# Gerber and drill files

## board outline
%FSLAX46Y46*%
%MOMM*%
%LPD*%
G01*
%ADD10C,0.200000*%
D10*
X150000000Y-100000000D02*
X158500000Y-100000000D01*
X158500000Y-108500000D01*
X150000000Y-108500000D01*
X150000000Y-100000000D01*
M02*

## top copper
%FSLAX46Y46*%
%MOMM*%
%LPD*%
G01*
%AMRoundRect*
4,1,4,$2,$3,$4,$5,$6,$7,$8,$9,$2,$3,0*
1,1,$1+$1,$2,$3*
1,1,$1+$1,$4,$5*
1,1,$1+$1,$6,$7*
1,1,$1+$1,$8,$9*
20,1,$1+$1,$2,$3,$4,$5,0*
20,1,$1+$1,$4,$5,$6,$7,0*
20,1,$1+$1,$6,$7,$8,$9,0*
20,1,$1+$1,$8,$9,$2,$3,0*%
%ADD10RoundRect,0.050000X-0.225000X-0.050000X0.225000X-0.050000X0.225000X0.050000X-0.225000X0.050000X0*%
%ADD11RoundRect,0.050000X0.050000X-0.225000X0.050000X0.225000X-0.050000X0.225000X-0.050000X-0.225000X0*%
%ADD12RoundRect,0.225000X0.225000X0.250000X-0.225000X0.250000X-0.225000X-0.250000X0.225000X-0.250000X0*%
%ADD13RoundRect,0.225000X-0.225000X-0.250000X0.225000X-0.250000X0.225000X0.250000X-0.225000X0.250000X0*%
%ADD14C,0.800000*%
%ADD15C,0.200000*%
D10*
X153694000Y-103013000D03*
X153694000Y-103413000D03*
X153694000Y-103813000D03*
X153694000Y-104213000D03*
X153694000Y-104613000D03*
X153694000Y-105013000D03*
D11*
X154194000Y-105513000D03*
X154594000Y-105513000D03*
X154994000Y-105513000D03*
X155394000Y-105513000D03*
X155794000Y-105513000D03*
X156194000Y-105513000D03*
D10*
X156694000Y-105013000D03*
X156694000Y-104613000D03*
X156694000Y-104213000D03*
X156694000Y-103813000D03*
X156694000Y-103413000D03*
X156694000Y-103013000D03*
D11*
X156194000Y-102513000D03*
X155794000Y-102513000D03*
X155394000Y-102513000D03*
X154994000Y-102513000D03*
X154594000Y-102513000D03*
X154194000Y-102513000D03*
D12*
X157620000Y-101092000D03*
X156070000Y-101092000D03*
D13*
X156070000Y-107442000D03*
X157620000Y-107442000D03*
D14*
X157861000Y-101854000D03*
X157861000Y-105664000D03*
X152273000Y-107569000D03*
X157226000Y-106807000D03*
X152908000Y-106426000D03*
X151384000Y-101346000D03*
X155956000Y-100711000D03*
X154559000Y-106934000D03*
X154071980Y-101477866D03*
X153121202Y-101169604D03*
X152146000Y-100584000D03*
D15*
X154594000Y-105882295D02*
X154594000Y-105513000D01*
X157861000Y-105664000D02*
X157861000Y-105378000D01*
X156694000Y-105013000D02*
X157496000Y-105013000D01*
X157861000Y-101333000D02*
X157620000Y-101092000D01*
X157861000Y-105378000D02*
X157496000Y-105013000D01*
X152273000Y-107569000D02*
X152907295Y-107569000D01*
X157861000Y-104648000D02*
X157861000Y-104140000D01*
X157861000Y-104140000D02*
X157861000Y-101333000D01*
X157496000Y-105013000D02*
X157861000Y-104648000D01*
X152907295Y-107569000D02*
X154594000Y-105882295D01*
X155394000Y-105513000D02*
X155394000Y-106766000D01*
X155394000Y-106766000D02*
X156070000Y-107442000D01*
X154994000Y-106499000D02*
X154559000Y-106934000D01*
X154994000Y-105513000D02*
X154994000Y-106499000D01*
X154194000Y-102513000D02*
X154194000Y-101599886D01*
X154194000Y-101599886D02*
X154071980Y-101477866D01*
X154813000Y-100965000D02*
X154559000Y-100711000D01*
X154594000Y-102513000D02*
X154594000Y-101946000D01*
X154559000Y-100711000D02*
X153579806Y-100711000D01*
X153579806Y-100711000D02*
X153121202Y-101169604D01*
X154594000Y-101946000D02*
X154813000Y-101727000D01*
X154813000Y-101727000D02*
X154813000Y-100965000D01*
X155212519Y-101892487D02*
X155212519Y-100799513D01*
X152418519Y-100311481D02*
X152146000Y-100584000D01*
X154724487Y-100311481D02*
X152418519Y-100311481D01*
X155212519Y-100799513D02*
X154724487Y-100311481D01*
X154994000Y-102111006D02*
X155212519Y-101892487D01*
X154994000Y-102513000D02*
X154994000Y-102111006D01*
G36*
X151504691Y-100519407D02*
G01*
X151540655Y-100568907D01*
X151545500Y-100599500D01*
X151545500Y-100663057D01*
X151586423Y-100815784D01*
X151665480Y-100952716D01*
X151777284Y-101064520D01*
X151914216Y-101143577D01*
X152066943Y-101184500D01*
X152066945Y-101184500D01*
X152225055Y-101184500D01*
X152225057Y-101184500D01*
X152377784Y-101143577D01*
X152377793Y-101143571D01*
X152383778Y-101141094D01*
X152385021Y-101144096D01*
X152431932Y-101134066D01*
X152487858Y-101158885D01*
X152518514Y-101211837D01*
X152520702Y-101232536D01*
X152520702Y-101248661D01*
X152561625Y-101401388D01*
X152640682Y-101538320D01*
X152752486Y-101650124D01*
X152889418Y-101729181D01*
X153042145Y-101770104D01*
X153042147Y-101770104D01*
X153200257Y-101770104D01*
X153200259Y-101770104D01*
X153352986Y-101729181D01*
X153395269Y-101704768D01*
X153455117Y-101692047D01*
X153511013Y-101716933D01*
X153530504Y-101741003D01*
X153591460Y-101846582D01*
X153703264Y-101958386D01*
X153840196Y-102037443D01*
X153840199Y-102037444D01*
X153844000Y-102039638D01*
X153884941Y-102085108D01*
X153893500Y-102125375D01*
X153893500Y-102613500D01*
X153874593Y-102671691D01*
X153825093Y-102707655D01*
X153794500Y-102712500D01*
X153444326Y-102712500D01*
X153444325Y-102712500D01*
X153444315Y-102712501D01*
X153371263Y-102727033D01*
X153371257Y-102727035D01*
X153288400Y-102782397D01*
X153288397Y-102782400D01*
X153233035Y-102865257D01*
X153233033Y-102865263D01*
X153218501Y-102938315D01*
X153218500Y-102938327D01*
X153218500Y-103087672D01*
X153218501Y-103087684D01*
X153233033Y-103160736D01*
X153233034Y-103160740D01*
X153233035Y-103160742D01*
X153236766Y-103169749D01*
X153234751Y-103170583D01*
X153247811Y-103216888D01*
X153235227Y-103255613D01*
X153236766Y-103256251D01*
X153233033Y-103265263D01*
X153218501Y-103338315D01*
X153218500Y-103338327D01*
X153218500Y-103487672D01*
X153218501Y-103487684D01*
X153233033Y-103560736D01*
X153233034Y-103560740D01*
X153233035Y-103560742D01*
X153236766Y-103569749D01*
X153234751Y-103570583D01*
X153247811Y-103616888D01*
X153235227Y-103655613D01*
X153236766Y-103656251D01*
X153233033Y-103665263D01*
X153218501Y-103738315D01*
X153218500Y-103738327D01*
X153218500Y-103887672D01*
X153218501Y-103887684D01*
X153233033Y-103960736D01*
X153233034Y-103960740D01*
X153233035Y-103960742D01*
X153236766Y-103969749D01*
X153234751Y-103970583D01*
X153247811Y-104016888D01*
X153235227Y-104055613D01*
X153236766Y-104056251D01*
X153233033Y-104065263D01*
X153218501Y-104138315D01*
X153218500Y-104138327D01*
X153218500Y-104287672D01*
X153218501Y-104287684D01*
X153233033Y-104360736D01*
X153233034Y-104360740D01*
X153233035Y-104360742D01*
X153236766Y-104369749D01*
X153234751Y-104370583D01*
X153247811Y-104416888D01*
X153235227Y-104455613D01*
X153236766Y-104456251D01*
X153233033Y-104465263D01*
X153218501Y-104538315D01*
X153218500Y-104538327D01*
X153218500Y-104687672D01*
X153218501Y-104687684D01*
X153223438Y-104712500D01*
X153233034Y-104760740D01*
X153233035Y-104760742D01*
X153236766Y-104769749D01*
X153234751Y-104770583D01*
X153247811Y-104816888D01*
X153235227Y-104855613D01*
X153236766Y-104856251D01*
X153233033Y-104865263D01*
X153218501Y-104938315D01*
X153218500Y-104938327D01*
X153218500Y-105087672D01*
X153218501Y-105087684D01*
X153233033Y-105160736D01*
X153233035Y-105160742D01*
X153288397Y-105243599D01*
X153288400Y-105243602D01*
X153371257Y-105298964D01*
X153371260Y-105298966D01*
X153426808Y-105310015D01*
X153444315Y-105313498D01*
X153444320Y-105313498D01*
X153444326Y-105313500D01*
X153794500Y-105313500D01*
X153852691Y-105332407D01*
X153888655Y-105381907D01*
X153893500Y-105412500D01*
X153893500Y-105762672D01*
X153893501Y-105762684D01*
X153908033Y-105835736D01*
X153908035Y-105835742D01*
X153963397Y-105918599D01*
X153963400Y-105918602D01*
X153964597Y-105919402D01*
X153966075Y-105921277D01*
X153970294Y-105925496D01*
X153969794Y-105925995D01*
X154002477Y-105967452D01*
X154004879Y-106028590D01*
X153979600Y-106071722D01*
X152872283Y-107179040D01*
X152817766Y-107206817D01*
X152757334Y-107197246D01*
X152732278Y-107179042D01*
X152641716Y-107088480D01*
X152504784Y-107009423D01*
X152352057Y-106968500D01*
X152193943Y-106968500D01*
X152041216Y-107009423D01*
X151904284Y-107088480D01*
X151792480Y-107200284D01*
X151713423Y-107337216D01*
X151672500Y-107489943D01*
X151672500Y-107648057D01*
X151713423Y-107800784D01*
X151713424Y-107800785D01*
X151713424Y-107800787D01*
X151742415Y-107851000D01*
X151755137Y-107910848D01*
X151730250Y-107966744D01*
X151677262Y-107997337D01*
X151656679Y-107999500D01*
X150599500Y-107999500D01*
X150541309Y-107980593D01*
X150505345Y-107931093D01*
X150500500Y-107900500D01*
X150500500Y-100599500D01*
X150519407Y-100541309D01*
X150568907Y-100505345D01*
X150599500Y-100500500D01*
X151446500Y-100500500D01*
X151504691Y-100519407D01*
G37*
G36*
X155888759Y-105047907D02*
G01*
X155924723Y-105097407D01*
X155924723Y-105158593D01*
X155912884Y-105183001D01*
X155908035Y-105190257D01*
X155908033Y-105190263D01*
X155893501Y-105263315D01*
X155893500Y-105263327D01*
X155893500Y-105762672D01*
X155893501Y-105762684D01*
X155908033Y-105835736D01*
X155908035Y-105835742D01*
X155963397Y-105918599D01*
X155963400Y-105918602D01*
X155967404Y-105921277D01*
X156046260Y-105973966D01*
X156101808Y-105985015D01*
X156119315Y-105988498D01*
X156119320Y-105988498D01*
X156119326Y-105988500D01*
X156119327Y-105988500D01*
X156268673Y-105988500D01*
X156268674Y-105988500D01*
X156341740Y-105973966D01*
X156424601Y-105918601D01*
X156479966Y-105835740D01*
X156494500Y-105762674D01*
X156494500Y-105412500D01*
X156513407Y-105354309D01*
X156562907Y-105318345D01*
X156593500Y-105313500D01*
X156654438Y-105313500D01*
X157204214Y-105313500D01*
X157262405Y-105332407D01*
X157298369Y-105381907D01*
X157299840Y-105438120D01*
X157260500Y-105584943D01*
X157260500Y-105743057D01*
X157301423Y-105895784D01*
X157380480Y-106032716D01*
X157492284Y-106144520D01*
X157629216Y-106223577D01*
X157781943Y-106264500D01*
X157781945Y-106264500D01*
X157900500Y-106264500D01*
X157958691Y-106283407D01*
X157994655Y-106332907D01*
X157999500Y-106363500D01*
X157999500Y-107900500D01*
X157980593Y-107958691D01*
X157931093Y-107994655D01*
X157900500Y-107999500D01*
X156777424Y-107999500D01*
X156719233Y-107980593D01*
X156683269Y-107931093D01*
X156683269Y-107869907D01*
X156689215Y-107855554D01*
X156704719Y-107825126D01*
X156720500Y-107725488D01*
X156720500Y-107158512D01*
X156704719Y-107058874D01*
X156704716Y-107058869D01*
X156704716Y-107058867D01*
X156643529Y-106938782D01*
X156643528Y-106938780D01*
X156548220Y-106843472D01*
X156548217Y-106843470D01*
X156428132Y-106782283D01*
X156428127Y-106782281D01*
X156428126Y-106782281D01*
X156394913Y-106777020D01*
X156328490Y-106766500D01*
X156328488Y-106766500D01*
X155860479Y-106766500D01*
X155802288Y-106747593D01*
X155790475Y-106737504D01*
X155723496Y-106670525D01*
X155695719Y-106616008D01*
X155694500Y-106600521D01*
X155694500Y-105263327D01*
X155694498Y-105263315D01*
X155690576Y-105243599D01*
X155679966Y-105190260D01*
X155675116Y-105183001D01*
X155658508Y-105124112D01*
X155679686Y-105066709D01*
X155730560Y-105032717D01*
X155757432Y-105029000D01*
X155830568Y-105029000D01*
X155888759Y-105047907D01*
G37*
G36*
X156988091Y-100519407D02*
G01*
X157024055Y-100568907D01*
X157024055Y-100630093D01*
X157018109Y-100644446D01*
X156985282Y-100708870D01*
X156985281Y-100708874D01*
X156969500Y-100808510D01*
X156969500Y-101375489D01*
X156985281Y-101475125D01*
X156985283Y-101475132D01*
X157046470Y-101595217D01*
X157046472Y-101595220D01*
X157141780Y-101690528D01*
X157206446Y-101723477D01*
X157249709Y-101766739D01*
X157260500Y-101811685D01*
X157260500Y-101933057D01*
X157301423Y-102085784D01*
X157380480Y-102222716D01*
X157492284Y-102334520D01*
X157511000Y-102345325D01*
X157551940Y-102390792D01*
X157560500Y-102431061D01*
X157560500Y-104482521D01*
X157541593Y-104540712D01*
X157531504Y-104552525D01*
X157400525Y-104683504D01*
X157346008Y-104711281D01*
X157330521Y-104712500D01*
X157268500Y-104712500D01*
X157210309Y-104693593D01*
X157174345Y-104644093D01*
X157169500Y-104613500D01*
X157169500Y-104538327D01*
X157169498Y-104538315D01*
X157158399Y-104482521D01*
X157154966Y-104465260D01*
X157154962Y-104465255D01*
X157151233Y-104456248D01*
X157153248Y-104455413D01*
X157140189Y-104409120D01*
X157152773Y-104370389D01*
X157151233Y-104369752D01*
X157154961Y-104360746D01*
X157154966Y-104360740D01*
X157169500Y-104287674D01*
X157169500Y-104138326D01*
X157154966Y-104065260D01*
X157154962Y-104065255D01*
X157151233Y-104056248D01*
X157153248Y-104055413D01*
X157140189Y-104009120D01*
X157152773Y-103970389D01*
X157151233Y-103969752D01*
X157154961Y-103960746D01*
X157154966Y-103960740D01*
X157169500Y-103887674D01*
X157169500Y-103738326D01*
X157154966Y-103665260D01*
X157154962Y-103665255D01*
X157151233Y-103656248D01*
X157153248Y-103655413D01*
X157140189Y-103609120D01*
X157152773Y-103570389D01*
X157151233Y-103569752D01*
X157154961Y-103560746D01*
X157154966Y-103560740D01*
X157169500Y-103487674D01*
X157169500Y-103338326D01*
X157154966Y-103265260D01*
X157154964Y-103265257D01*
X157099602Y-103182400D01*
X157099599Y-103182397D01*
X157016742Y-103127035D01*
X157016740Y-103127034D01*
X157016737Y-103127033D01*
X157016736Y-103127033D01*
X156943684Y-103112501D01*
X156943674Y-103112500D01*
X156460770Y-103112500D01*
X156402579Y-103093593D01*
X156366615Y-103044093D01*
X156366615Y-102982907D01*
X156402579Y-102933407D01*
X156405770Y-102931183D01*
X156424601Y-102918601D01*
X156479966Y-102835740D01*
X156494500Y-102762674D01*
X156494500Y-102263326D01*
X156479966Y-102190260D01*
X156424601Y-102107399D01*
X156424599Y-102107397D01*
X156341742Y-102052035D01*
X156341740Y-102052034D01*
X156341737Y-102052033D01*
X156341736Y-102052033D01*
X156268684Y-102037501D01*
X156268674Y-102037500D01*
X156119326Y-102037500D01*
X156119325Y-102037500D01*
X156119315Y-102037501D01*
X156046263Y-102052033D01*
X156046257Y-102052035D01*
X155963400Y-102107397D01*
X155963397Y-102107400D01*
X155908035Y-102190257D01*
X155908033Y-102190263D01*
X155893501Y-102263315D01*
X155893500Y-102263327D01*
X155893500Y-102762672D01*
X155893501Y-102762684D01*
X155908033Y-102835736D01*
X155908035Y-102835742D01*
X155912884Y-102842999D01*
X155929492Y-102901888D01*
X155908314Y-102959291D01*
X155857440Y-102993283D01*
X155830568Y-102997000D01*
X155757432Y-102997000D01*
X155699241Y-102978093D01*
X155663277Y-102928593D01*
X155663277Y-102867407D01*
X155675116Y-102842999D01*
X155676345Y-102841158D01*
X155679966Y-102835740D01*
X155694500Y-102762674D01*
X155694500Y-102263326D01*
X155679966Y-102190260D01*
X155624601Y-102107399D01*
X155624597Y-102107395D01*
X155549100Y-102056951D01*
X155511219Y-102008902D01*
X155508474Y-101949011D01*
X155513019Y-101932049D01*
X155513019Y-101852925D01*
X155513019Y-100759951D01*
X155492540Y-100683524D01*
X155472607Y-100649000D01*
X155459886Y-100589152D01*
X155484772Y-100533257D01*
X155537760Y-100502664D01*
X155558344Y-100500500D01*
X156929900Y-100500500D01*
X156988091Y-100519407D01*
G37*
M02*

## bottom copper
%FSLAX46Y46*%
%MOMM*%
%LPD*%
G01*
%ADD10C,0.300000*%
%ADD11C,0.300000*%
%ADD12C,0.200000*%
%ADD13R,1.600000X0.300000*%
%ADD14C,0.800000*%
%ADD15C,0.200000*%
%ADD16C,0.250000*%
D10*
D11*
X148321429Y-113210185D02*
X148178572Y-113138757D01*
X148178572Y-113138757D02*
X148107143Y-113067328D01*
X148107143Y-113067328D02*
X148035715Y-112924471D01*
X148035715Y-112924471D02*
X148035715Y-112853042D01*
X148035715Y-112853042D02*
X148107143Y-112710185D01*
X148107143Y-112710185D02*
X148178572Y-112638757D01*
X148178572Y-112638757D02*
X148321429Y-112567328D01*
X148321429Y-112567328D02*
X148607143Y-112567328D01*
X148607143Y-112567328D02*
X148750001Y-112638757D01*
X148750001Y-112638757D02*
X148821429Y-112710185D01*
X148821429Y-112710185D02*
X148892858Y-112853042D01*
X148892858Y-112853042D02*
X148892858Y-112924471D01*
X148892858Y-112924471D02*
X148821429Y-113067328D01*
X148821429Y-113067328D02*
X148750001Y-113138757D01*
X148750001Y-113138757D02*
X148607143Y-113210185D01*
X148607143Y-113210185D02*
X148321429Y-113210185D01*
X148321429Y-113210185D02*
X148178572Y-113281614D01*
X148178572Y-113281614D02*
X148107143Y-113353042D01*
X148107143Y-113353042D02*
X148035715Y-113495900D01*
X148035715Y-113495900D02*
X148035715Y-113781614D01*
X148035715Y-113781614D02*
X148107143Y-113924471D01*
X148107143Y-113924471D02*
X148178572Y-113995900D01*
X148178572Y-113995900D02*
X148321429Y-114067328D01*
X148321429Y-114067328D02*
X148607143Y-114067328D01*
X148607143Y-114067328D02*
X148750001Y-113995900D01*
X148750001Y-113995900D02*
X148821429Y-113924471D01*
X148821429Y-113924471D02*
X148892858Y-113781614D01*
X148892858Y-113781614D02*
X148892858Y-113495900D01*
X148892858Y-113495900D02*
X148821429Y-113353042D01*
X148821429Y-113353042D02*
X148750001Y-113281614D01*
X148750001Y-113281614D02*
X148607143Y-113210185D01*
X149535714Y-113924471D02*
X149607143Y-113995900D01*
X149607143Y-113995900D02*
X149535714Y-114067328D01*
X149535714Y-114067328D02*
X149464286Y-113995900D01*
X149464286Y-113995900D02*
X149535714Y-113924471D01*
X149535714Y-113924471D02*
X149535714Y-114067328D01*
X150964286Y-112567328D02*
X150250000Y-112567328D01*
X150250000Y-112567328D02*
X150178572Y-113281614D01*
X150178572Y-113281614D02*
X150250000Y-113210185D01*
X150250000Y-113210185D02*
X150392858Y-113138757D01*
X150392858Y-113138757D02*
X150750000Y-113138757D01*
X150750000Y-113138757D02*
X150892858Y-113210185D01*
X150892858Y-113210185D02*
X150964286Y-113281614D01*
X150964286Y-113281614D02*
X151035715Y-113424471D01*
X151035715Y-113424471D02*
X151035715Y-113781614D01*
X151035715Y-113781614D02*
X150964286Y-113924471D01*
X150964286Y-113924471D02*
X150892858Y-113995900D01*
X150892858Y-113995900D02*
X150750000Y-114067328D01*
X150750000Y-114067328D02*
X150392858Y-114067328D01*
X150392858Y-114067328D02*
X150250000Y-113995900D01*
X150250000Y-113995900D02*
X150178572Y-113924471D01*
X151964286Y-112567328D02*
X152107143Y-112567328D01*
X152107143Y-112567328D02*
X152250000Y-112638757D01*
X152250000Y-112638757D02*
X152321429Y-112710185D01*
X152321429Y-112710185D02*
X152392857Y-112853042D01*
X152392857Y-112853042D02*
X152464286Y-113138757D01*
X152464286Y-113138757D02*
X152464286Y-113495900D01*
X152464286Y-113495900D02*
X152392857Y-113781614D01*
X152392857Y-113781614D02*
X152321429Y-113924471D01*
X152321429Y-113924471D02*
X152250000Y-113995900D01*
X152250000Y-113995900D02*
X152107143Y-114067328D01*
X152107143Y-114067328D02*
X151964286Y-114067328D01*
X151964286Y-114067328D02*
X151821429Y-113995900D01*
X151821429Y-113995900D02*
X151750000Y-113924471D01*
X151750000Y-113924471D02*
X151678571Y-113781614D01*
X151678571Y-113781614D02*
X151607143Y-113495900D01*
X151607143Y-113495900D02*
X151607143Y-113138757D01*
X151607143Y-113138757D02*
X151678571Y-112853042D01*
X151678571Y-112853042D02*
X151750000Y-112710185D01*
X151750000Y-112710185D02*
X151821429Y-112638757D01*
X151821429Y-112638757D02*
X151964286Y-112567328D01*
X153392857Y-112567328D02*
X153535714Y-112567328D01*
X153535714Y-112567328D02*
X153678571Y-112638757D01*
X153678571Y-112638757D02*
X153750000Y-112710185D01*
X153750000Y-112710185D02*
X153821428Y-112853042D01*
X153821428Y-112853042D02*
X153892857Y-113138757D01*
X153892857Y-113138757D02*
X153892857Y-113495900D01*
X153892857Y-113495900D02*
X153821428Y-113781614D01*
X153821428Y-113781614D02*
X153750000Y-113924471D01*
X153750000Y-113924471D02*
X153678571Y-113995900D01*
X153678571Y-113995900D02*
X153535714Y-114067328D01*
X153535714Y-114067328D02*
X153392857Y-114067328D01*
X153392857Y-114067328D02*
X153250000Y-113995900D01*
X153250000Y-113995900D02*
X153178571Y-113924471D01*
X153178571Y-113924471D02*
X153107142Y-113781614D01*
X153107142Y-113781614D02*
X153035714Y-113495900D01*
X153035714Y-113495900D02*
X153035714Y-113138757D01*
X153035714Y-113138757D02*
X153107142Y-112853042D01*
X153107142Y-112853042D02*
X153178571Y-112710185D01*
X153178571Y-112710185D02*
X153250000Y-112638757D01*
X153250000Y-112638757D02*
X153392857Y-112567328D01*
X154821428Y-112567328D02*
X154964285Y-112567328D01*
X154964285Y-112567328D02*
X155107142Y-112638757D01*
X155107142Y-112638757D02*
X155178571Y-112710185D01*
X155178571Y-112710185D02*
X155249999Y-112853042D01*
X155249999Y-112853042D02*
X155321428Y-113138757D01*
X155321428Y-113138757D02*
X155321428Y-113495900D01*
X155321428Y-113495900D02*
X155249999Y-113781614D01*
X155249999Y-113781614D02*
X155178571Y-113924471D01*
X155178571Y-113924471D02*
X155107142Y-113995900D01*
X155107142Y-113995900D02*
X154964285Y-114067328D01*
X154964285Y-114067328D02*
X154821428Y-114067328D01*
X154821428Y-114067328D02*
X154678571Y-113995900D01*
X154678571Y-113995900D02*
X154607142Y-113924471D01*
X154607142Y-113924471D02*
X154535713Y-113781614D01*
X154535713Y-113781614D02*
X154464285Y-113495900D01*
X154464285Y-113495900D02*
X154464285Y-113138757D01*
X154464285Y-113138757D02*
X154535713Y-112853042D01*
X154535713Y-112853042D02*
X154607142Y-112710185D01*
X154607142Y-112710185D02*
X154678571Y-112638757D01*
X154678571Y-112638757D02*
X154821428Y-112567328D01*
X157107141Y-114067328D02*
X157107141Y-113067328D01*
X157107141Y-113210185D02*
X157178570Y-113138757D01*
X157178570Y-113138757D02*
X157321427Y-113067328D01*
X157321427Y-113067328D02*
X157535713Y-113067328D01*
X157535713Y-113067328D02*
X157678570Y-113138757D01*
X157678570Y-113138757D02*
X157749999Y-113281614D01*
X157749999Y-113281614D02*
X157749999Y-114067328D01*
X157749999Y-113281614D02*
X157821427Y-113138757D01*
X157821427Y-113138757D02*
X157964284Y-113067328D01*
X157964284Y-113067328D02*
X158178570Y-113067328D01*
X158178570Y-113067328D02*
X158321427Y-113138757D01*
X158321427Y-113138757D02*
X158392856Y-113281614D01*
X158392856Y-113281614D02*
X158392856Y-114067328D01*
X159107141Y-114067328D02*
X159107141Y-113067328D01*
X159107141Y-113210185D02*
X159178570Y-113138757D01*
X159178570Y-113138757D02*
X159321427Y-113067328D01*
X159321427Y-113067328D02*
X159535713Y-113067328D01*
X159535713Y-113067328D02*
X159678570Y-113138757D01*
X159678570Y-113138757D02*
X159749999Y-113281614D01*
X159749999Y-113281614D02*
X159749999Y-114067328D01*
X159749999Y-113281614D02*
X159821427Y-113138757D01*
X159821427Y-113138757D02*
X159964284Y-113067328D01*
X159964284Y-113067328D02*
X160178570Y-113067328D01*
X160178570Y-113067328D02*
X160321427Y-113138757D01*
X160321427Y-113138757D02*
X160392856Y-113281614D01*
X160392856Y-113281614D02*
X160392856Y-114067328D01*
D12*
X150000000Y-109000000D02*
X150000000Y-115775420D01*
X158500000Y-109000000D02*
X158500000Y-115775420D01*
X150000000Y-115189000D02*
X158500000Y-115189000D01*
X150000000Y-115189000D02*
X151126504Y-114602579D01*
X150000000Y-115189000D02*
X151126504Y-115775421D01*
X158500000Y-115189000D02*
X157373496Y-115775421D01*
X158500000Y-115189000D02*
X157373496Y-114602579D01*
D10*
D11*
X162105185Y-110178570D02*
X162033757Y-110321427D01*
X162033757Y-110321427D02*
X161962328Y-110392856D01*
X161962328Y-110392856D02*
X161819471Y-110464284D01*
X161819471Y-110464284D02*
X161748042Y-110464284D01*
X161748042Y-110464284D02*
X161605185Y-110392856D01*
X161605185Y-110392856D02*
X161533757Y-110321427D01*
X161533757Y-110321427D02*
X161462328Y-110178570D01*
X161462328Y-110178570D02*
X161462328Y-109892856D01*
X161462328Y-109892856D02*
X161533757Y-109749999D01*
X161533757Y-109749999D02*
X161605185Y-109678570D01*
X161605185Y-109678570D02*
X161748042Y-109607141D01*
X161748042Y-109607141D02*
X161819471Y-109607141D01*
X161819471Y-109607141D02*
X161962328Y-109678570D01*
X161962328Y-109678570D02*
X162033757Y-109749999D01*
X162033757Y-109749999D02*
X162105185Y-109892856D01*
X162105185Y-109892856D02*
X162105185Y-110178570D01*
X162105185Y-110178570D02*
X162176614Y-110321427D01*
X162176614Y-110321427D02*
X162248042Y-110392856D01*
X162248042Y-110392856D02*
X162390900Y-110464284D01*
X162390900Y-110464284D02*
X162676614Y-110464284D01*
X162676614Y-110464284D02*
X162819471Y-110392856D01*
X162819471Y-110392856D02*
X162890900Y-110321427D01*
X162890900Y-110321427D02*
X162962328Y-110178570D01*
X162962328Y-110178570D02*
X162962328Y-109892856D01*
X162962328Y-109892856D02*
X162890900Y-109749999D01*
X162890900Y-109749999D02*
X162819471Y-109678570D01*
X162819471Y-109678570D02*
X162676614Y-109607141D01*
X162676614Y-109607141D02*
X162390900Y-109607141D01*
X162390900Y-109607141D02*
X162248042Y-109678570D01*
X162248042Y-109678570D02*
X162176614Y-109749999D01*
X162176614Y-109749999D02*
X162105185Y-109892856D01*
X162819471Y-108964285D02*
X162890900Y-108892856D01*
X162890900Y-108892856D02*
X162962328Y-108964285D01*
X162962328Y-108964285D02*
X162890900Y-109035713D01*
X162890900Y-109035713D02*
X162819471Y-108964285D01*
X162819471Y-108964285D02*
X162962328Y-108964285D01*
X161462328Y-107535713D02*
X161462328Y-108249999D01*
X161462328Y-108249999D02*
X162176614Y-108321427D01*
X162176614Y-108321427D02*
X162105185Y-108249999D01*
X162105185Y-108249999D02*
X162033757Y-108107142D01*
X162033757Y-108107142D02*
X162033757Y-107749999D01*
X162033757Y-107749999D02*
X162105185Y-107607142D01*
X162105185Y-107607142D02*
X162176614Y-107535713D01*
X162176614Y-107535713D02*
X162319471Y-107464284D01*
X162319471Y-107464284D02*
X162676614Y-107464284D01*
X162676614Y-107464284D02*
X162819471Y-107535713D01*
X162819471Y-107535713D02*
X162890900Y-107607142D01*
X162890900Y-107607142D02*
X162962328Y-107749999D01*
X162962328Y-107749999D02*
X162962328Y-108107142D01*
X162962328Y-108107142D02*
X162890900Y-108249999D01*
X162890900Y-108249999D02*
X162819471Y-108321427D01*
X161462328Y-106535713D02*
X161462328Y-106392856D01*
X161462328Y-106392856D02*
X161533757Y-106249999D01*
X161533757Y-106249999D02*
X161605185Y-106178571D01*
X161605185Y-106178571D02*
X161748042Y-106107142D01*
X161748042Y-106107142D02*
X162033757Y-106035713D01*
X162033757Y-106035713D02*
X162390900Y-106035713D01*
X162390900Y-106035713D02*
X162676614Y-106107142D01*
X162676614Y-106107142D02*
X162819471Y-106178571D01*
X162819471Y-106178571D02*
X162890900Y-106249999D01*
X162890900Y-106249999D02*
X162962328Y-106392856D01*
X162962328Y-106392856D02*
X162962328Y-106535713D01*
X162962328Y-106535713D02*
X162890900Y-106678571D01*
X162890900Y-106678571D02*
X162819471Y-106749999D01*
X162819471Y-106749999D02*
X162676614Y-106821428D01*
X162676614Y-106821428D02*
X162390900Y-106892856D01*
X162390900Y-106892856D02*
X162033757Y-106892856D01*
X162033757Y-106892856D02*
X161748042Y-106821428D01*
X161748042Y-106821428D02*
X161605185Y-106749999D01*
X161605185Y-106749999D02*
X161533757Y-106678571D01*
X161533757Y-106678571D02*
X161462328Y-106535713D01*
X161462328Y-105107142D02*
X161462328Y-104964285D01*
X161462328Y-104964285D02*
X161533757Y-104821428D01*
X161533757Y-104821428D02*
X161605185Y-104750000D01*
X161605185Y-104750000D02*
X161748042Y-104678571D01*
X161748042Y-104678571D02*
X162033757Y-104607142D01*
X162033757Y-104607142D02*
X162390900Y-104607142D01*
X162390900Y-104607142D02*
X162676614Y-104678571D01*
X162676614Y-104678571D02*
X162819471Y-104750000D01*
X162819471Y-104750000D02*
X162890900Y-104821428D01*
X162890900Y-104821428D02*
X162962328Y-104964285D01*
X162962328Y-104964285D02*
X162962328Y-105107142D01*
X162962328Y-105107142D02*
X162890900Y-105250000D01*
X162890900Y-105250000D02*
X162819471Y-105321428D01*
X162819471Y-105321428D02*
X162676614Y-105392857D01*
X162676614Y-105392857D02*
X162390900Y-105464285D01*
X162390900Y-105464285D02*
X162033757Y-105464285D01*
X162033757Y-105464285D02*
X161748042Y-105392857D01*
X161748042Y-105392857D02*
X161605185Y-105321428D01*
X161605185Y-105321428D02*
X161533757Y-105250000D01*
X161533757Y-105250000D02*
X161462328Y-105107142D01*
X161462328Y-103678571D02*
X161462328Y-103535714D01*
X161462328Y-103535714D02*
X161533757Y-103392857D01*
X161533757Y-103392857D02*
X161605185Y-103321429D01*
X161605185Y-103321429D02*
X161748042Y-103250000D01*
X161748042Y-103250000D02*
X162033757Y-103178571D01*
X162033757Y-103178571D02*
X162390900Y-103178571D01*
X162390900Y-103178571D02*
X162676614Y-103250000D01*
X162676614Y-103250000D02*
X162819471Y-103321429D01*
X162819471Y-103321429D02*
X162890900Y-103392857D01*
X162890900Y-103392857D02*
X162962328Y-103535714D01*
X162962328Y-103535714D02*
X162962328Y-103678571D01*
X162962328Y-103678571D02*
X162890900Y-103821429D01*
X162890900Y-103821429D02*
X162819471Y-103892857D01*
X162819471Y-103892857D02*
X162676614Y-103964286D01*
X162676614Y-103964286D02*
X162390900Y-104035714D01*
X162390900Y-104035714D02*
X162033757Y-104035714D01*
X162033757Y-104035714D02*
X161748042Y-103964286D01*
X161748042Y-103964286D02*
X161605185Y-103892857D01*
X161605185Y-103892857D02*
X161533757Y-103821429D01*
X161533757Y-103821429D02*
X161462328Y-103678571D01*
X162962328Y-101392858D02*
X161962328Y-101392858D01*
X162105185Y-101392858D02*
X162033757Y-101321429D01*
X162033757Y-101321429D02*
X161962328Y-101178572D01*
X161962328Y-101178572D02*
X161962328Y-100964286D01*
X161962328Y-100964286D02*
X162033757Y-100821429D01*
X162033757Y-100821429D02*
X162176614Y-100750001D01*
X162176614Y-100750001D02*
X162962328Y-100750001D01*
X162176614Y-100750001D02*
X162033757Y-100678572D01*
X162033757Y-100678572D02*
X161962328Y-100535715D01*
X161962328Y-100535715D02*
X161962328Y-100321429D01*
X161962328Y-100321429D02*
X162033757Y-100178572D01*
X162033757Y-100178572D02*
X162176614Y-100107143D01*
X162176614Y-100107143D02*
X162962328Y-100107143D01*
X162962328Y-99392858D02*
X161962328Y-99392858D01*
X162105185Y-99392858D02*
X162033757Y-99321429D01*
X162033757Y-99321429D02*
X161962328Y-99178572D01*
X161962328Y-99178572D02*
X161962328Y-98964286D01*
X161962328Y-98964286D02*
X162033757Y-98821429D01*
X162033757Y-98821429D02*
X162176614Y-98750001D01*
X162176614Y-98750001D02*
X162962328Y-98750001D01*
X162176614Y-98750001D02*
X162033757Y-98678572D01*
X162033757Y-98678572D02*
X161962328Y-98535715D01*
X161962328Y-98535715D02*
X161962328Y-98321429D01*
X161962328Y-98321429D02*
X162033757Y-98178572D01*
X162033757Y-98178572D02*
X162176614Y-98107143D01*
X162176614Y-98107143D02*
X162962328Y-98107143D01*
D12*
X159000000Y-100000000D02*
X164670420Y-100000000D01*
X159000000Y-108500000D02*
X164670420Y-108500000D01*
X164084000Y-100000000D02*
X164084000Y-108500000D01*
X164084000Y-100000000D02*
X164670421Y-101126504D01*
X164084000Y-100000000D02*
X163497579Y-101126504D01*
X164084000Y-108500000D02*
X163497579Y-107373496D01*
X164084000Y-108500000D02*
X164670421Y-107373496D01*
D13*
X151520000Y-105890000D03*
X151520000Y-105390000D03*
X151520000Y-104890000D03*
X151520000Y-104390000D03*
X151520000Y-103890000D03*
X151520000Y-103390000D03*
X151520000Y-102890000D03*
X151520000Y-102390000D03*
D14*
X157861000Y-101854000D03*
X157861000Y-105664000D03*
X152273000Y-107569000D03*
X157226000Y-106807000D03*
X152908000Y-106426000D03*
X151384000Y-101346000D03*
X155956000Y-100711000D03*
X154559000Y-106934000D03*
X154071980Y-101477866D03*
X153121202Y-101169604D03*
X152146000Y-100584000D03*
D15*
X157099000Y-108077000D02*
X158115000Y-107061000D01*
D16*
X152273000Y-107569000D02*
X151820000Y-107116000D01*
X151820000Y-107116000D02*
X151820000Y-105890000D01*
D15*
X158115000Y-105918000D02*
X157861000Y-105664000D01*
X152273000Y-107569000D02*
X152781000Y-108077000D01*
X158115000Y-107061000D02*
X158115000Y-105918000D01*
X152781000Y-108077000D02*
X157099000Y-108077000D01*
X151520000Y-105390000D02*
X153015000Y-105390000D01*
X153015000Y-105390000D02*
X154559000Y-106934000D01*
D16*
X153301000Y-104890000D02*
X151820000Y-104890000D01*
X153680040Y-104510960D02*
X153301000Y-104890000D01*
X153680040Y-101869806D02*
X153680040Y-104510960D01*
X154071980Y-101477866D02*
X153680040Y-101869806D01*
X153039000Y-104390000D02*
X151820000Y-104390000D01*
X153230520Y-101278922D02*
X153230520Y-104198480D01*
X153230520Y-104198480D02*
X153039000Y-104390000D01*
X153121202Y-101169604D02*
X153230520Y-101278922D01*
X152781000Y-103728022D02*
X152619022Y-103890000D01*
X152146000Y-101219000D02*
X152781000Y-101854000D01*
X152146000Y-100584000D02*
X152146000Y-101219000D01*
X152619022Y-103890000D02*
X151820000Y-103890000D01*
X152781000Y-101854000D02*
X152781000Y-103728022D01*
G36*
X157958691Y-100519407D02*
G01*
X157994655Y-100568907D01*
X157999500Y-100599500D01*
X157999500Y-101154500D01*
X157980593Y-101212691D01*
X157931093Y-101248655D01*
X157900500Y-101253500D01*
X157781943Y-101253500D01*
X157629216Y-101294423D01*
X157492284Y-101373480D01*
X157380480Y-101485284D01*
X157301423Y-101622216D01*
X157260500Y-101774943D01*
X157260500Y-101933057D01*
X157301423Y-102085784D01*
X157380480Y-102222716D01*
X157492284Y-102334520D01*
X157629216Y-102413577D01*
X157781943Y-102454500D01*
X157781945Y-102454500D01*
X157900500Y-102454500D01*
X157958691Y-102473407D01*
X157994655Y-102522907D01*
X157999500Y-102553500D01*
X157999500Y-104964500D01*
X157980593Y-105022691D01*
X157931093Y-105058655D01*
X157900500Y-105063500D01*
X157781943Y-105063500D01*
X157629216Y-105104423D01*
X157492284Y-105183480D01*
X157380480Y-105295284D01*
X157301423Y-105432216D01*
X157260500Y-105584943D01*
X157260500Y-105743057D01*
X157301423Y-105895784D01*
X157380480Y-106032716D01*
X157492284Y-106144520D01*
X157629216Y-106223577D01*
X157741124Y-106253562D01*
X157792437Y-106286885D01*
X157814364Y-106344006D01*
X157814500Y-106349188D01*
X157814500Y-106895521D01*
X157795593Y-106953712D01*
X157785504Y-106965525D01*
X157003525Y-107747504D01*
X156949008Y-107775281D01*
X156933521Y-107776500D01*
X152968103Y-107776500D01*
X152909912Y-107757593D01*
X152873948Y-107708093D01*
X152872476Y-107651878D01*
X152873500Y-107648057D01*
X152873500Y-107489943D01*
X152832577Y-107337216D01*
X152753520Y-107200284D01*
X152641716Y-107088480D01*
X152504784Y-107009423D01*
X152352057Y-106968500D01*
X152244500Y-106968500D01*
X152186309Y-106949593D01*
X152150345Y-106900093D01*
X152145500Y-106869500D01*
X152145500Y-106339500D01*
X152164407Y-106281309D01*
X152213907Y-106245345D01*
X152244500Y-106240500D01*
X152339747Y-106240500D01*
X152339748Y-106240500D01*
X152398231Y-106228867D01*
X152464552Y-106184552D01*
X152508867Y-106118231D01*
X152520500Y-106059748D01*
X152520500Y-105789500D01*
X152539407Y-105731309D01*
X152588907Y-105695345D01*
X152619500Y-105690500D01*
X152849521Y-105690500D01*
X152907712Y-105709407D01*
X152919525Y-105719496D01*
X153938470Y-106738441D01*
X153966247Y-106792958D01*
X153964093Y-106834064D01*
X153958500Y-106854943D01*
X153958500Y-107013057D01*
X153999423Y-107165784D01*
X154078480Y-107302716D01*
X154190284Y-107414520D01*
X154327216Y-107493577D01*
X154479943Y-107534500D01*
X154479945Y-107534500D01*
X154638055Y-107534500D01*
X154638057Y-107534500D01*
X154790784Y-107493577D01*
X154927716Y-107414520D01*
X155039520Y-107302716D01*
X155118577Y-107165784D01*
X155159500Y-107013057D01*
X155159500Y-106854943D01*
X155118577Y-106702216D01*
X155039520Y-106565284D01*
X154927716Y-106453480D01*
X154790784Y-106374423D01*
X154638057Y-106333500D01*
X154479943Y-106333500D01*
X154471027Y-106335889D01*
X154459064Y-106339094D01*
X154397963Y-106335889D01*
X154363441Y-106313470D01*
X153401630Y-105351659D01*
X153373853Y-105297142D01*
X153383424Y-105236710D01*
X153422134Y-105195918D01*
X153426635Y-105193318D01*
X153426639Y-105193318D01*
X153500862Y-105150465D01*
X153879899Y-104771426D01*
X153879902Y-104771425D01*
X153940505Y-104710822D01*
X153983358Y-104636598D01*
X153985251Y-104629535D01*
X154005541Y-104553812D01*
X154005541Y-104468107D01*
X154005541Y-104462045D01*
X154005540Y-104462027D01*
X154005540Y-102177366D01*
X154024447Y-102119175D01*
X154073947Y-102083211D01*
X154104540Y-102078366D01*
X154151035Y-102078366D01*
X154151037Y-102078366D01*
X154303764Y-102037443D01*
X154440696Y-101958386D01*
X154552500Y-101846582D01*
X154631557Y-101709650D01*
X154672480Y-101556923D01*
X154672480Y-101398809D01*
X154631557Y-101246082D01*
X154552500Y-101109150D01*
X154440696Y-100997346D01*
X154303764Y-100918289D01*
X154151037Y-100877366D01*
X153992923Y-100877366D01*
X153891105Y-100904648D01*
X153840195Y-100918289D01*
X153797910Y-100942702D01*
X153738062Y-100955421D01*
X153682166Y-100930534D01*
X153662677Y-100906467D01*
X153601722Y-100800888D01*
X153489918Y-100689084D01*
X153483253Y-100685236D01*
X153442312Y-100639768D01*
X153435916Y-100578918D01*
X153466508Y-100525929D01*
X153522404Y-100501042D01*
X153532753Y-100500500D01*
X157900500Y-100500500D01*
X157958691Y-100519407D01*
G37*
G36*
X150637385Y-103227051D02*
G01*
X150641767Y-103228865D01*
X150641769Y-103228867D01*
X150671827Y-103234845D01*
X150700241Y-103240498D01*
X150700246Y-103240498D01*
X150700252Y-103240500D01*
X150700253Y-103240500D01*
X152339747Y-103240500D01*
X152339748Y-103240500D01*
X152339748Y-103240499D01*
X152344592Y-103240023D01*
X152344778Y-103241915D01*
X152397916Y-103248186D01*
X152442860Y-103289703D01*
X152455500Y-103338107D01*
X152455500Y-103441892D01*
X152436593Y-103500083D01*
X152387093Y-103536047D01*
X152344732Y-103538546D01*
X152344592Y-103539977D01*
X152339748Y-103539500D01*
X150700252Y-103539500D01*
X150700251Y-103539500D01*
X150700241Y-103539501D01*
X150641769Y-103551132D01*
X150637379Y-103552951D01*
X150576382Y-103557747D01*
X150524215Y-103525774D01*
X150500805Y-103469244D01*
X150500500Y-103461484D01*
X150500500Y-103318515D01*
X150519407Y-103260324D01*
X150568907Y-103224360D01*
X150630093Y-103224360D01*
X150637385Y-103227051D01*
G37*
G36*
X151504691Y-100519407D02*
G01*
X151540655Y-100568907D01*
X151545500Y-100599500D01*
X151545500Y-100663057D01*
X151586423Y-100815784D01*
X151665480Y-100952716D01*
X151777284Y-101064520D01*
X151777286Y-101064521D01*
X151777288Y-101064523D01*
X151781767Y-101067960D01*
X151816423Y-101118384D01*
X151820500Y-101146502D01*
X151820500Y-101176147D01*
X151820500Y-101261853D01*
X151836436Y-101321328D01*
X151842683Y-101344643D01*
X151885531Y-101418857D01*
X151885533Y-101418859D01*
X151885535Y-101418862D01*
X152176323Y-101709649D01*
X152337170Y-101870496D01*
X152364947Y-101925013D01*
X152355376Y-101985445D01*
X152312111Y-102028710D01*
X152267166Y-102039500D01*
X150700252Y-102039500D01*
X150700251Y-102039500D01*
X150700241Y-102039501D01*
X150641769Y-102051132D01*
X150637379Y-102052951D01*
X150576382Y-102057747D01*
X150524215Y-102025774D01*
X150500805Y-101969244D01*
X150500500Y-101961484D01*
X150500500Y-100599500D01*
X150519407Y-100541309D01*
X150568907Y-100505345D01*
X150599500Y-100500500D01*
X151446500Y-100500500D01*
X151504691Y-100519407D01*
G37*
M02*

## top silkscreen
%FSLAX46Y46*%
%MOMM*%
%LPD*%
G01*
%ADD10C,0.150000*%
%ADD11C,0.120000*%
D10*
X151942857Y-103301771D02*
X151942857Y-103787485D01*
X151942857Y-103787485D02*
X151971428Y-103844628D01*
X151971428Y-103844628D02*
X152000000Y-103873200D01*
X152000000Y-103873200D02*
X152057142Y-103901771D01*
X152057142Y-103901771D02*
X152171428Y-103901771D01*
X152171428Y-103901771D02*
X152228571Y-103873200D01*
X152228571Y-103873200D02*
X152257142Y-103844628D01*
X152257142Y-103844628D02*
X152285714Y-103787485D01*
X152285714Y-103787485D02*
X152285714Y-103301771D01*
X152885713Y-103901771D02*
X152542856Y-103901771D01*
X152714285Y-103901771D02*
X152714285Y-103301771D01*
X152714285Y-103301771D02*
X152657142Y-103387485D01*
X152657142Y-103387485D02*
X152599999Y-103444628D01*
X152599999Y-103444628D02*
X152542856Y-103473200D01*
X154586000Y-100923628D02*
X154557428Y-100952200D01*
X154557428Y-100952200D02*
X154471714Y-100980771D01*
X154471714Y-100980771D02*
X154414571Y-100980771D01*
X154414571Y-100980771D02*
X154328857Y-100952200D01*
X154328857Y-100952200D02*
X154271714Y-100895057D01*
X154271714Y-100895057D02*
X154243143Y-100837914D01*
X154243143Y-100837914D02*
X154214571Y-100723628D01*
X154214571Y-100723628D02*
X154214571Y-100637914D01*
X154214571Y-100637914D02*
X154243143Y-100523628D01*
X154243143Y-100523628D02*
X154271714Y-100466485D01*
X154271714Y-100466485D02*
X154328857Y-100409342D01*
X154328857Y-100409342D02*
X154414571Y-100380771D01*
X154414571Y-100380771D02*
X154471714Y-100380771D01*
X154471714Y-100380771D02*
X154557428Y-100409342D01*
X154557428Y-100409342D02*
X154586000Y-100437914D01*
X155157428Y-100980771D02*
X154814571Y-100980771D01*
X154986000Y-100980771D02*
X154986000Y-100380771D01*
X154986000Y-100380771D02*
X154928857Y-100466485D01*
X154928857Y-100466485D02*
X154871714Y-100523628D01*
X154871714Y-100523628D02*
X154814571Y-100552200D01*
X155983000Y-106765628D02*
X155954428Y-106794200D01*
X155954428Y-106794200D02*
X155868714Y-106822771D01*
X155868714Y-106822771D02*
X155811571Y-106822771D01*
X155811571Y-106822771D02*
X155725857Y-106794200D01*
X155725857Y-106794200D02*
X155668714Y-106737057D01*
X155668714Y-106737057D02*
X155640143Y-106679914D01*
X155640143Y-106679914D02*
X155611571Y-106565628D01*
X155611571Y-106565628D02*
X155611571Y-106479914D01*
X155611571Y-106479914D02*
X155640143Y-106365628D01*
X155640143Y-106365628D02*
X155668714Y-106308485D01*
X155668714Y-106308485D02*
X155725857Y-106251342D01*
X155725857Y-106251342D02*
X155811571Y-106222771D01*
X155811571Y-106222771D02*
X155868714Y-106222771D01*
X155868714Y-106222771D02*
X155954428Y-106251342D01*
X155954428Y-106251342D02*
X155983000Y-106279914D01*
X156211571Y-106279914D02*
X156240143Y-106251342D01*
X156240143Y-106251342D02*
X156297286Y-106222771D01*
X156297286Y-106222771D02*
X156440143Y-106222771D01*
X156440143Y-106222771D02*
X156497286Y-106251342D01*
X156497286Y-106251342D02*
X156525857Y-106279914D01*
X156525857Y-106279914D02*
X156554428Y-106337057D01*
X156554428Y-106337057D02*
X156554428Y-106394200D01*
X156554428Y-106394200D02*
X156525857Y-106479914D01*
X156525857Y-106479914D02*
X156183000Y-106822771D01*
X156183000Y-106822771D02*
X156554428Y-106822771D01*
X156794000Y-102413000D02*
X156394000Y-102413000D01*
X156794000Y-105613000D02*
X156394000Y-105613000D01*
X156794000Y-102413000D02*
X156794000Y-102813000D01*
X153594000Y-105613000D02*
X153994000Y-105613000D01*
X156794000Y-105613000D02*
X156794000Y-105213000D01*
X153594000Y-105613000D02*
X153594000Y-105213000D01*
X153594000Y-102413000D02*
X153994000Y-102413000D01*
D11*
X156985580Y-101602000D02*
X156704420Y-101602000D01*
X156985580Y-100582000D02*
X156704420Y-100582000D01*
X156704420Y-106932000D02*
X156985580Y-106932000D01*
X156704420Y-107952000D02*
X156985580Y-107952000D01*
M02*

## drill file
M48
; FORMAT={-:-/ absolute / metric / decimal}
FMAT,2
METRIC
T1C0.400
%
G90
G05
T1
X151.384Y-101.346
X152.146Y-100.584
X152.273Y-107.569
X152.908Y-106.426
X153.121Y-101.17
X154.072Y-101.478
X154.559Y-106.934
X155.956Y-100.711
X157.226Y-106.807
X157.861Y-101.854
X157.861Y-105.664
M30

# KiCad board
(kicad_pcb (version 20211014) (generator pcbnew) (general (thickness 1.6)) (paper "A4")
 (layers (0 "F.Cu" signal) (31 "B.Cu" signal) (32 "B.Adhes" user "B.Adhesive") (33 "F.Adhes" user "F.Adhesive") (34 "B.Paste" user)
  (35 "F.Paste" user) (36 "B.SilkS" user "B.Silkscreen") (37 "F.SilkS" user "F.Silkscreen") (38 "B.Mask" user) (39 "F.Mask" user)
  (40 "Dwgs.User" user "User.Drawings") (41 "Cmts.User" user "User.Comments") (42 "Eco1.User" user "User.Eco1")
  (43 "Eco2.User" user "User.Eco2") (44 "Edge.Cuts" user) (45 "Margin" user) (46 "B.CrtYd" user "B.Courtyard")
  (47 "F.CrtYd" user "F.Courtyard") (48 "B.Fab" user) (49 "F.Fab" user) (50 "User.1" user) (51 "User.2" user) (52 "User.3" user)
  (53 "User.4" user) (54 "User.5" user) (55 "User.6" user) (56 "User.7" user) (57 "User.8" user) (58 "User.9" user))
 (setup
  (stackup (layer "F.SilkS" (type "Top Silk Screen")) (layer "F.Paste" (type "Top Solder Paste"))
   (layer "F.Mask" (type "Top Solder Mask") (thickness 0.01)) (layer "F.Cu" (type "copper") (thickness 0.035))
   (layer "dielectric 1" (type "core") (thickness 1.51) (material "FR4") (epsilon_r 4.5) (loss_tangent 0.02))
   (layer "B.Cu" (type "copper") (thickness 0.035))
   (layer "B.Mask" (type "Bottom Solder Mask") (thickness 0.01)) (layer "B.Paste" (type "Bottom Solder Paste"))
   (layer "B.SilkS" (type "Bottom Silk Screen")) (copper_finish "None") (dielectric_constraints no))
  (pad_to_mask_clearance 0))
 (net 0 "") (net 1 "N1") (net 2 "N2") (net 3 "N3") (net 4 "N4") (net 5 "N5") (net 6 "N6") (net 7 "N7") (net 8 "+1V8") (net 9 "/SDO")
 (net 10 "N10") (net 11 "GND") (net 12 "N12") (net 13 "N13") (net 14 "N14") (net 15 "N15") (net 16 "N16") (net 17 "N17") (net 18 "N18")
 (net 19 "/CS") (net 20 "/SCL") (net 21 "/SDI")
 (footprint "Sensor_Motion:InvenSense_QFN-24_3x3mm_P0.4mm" (layer "F.Cu") (at 155.194 104.013)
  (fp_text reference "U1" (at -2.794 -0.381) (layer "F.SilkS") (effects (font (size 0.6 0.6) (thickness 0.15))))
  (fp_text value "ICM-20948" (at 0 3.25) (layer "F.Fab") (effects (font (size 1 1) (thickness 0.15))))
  (fp_line (start 1.6 -1.6) (end 1.2 -1.6) (layer "F.SilkS") (width 0.15))
  (fp_line (start 1.6 1.6) (end 1.2 1.6) (layer "F.SilkS") (width 0.15))
  (fp_line (start 1.6 -1.6) (end 1.6 -1.2) (layer "F.SilkS") (width 0.15))
  (fp_line (start -1.6 1.6) (end -1.2 1.6) (layer "F.SilkS") (width 0.15))
  (fp_line (start 1.6 1.6) (end 1.6 1.2) (layer "F.SilkS") (width 0.15))
  (fp_line (start -1.6 1.6) (end -1.6 1.2) (layer "F.SilkS") (width 0.15))
  (fp_line (start -1.6 -1.6) (end -1.2 -1.6) (layer "F.SilkS") (width 0.15))
  (pad "1" smd roundrect (at -1.5 -1) (size 0.55 0.2) (layers "F.Cu" "F.Paste" "F.Mask") (roundrect_rratio 0.25) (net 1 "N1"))
  (pad "2" smd roundrect (at -1.5 -0.6) (size 0.55 0.2) (layers "F.Cu" "F.Paste" "F.Mask") (roundrect_rratio 0.25) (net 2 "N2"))
  (pad "3" smd roundrect (at -1.5 -0.2) (size 0.55 0.2) (layers "F.Cu" "F.Paste" "F.Mask") (roundrect_rratio 0.25) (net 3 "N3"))
  (pad "4" smd roundrect (at -1.5 0.2) (size 0.55 0.2) (layers "F.Cu" "F.Paste" "F.Mask") (roundrect_rratio 0.25) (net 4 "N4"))
  (pad "5" smd roundrect (at -1.5 0.6) (size 0.55 0.2) (layers "F.Cu" "F.Paste" "F.Mask") (roundrect_rratio 0.25) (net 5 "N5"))
  (pad "6" smd roundrect (at -1.5 1) (size 0.55 0.2) (layers "F.Cu" "F.Paste" "F.Mask") (roundrect_rratio 0.25) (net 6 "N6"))
  (pad "7" smd roundrect (at -1 1.5 90) (size 0.55 0.2) (layers "F.Cu" "F.Paste" "F.Mask") (roundrect_rratio 0.25) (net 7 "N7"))
  (pad "8" smd roundrect (at -0.6 1.5 90) (size 0.55 0.2) (layers "F.Cu" "F.Paste" "F.Mask") (roundrect_rratio 0.25) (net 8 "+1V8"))
  (pad "9" smd roundrect (at -0.2 1.5 90) (size 0.55 0.2) (layers "F.Cu" "F.Paste" "F.Mask") (roundrect_rratio 0.25) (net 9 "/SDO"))
  (pad "10" smd roundrect (at 0.2 1.5 90) (size 0.55 0.2) (layers "F.Cu" "F.Paste" "F.Mask") (roundrect_rratio 0.25) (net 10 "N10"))
  (pad "11" smd roundrect (at 0.6 1.5 90) (size 0.55 0.2) (layers "F.Cu" "F.Paste" "F.Mask") (roundrect_rratio 0.25) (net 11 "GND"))
  (pad "12" smd roundrect (at 1 1.5 90) (size 0.55 0.2) (layers "F.Cu" "F.Paste" "F.Mask") (roundrect_rratio 0.25) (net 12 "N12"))
  (pad "13" smd roundrect (at 1.5 1) (size 0.55 0.2) (layers "F.Cu" "F.Paste" "F.Mask") (roundrect_rratio 0.25) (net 8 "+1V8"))
  (pad "14" smd roundrect (at 1.5 0.6) (size 0.55 0.2) (layers "F.Cu" "F.Paste" "F.Mask") (roundrect_rratio 0.25) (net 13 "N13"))
  (pad "15" smd roundrect (at 1.5 0.2) (size 0.55 0.2) (layers "F.Cu" "F.Paste" "F.Mask") (roundrect_rratio 0.25) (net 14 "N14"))
  (pad "16" smd roundrect (at 1.5 -0.2) (size 0.55 0.2) (layers "F.Cu" "F.Paste" "F.Mask") (roundrect_rratio 0.25) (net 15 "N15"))
  (pad "17" smd roundrect (at 1.5 -0.6) (size 0.55 0.2) (layers "F.Cu" "F.Paste" "F.Mask") (roundrect_rratio 0.25) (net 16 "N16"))
  (pad "18" smd roundrect (at 1.5 -1) (size 0.55 0.2) (layers "F.Cu" "F.Paste" "F.Mask") (roundrect_rratio 0.25) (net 11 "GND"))
  (pad "19" smd roundrect (at 1 -1.5 90) (size 0.55 0.2) (layers "F.Cu" "F.Paste" "F.Mask") (roundrect_rratio 0.25) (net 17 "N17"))
  (pad "20" smd roundrect (at 0.6 -1.5 90) (size 0.55 0.2) (layers "F.Cu" "F.Paste" "F.Mask") (roundrect_rratio 0.25) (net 11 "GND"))
  (pad "21" smd roundrect (at 0.2 -1.5 90) (size 0.55 0.2) (layers "F.Cu" "F.Paste" "F.Mask") (roundrect_rratio 0.25) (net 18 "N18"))
  (pad "22" smd roundrect (at -0.2 -1.5 90) (size 0.55 0.2) (layers "F.Cu" "F.Paste" "F.Mask") (roundrect_rratio 0.25) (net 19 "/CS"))
  (pad "23" smd roundrect (at -0.6 -1.5 90) (size 0.55 0.2) (layers "F.Cu" "F.Paste" "F.Mask") (roundrect_rratio 0.25) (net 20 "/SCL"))
  (pad "24" smd roundrect (at -1 -1.5 90) (size 0.55 0.2) (layers "F.Cu" "F.Paste" "F.Mask") (roundrect_rratio 0.25) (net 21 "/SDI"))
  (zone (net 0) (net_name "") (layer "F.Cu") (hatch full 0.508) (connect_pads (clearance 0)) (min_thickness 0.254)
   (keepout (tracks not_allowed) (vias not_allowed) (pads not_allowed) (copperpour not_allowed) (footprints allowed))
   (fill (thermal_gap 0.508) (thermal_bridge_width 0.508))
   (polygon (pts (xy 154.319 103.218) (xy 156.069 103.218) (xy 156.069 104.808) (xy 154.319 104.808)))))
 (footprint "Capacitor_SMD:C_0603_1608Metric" (layer "F.Cu") (at 156.845 101.092 180)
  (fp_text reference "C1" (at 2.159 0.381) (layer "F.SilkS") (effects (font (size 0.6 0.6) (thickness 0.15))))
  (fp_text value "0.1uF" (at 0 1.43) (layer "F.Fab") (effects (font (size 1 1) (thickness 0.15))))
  (fp_line (start -0.14058 -0.51) (end 0.14058 -0.51) (layer "F.SilkS") (width 0.12))
  (fp_line (start -0.14058 0.51) (end 0.14058 0.51) (layer "F.SilkS") (width 0.12))
  (pad "1" smd roundrect (at -0.775 0 180) (size 0.9 0.95) (layers "F.Cu" "F.Paste" "F.Mask") (roundrect_rratio 0.25) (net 8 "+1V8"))
  (pad "2" smd roundrect (at 0.775 0 180) (size 0.9 0.95) (layers "F.Cu" "F.Paste" "F.Mask") (roundrect_rratio 0.25) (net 11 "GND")))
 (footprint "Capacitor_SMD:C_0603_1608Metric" (layer "F.Cu") (at 156.845 107.442)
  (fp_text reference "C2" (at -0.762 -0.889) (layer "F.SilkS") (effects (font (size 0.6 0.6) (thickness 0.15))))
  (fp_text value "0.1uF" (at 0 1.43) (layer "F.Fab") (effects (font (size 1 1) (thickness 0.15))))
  (fp_line (start -0.14058 -0.51) (end 0.14058 -0.51) (layer "F.SilkS") (width 0.12))
  (fp_line (start -0.14058 0.51) (end 0.14058 0.51) (layer "F.SilkS") (width 0.12))
  (pad "1" smd roundrect (at -0.775 0) (size 0.9 0.95) (layers "F.Cu" "F.Paste" "F.Mask") (roundrect_rratio 0.25) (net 10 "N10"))
  (pad "2" smd roundrect (at 0.775 0) (size 0.9 0.95) (layers "F.Cu" "F.Paste" "F.Mask") (roundrect_rratio 0.25) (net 11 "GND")))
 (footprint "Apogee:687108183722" (layer "B.Cu") (at 149.92 104.14 90)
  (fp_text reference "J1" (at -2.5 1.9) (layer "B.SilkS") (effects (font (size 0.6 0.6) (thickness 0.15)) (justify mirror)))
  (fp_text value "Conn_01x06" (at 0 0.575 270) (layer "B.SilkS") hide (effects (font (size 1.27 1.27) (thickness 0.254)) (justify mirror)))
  (pad "1" smd rect (at -1.75 1.6 90) (size 0.3 1.6) (layers "B.Cu" "B.Paste" "B.Mask") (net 8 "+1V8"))
  (pad "2" smd rect (at -1.25 1.6 90) (size 0.3 1.6) (layers "B.Cu" "B.Paste" "B.Mask") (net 9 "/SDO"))
  (pad "3" smd rect (at -0.75 1.6 90) (size 0.3 1.6) (layers "B.Cu" "B.Paste" "B.Mask") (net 21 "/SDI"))
  (pad "4" smd rect (at -0.25 1.6 90) (size 0.3 1.6) (layers "B.Cu" "B.Paste" "B.Mask") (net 20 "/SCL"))
  (pad "5" smd rect (at 0.25 1.6 90) (size 0.3 1.6) (layers "B.Cu" "B.Paste" "B.Mask") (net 19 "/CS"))
  (pad "6" smd rect (at 0.75 1.6 90) (size 0.3 1.6) (layers "B.Cu" "B.Paste" "B.Mask") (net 11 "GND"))
  (pad "7" smd rect (at 1.25 1.6 90) (size 0.3 1.6) (layers "B.Cu" "B.Paste" "B.Mask"))
  (pad "8" smd rect (at 1.75 1.6 90) (size 0.3 1.6) (layers "B.Cu" "B.Paste" "B.Mask")))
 (gr_rect (start 150 100) (end 158.5 108.5) (layer "Edge.Cuts") (width 0.2) (fill none))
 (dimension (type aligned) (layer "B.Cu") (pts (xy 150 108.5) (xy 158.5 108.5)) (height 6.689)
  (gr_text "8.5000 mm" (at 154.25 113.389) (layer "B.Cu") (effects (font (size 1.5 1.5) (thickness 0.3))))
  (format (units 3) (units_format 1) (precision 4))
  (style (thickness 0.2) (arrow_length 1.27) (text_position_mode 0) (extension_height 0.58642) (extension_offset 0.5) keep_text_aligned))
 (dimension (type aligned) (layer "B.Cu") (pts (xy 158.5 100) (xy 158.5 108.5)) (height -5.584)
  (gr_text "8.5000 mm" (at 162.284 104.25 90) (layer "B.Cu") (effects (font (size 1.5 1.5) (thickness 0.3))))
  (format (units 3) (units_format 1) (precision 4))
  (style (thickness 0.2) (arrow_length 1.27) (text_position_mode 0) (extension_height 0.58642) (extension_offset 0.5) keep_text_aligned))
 (segment (start 154.594 105.882295) (end 154.594 105.513) (width 0.2) (layer "F.Cu") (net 8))
 (segment (start 157.861 105.664) (end 157.861 105.378) (width 0.2) (layer "F.Cu") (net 8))
 (segment (start 156.694 105.013) (end 157.496 105.013) (width 0.2) (layer "F.Cu") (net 8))
 (segment (start 157.861 101.333) (end 157.62 101.092) (width 0.2) (layer "F.Cu") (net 8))
 (segment (start 157.861 105.378) (end 157.496 105.013) (width 0.2) (layer "F.Cu") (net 8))
 (segment (start 152.273 107.569) (end 152.907295 107.569) (width 0.2) (layer "F.Cu") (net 8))
 (segment (start 157.861 104.648) (end 157.861 104.14) (width 0.2) (layer "F.Cu") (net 8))
 (segment (start 157.861 104.14) (end 157.861 101.333) (width 0.2) (layer "F.Cu") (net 8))
 (segment (start 157.496 105.013) (end 157.861 104.648) (width 0.2) (layer "F.Cu") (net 8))
 (segment (start 152.907295 107.569) (end 154.594 105.882295) (width 0.2) (layer "F.Cu") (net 8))
 (via (at 157.861 101.854) (size 0.8) (drill 0.4) (layers "F.Cu" "B.Cu") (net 8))
 (via (at 157.861 105.664) (size 0.8) (drill 0.4) (layers "F.Cu" "B.Cu") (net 8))
 (via (at 152.273 107.569) (size 0.8) (drill 0.4) (layers "F.Cu" "B.Cu") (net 8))
 (segment (start 157.099 108.077) (end 158.115 107.061) (width 0.2) (layer "B.Cu") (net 8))
 (segment (start 152.273 107.569) (end 151.82 107.116) (width 0.25) (layer "B.Cu") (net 8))
 (segment (start 151.82 107.116) (end 151.82 105.89) (width 0.25) (layer "B.Cu") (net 8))
 (segment (start 158.115 105.918) (end 157.861 105.664) (width 0.2) (layer "B.Cu") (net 8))
 (segment (start 152.273 107.569) (end 152.781 108.077) (width 0.2) (layer "B.Cu") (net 8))
 (segment (start 158.115 107.061) (end 158.115 105.918) (width 0.2) (layer "B.Cu") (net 8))
 (segment (start 152.781 108.077) (end 157.099 108.077) (width 0.2) (layer "B.Cu") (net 8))
 (via (at 157.226 106.807) (size 0.8) (drill 0.4) (layers "F.Cu" "B.Cu") (free) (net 11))
 (via (at 152.908 106.426) (size 0.8) (drill 0.4) (layers "F.Cu" "B.Cu") (free) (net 11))
 (via (at 151.384 101.346) (size 0.8) (drill 0.4) (layers "F.Cu" "B.Cu") (free) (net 11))
 (via (at 155.956 100.711) (size 0.8) (drill 0.4) (layers "F.Cu" "B.Cu") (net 11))
 (segment (start 155.394 105.513) (end 155.394 106.766) (width 0.2) (layer "F.Cu") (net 10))
 (segment (start 155.394 106.766) (end 156.07 107.442) (width 0.2) (layer "F.Cu") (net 10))
 (segment (start 154.994 106.499) (end 154.559 106.934) (width 0.2) (layer "F.Cu") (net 9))
 (segment (start 154.994 105.513) (end 154.994 106.499) (width 0.2) (layer "F.Cu") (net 9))
 (via (at 154.559 106.934) (size 0.8) (drill 0.4) (layers "F.Cu" "B.Cu") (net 9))
 (segment (start 151.52 105.39) (end 153.015 105.39) (width 0.2) (layer "B.Cu") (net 9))
 (segment (start 153.015 105.39) (end 154.559 106.934) (width 0.2) (layer "B.Cu") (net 9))
 (segment (start 154.194 102.513) (end 154.194 101.599886) (width 0.2) (layer "F.Cu") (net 21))
 (segment (start 154.194 101.599886) (end 154.07198 101.477866) (width 0.2) (layer "F.Cu") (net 21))
 (via (at 154.07198 101.477866) (size 0.8) (drill 0.4) (layers "F.Cu" "B.Cu") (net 21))
 (segment (start 153.301 104.89) (end 151.82 104.89) (width 0.25) (layer "B.Cu") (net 21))
 (segment (start 153.68004 104.51096) (end 153.301 104.89) (width 0.25) (layer "B.Cu") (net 21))
 (segment (start 153.68004 101.869806) (end 153.68004 104.51096) (width 0.25) (layer "B.Cu") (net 21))
 (segment (start 154.07198 101.477866) (end 153.68004 101.869806) (width 0.25) (layer "B.Cu") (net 21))
 (segment (start 154.813 100.965) (end 154.559 100.711) (width 0.2) (layer "F.Cu") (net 20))
 (segment (start 154.594 102.513) (end 154.594 101.946) (width 0.2) (layer "F.Cu") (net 20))
 (segment (start 154.559 100.711) (end 153.579806 100.711) (width 0.2) (layer "F.Cu") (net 20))
 (segment (start 153.579806 100.711) (end 153.121202 101.169604) (width 0.2) (layer "F.Cu") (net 20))
 (segment (start 154.594 101.946) (end 154.813 101.727) (width 0.2) (layer "F.Cu") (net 20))
 (segment (start 154.813 101.727) (end 154.813 100.965) (width 0.2) (layer "F.Cu") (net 20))
 (via (at 153.121202 101.169604) (size 0.8) (drill 0.4) (layers "F.Cu" "B.Cu") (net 20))
 (segment (start 153.039 104.39) (end 151.82 104.39) (width 0.25) (layer "B.Cu") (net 20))
 (segment (start 153.23052 101.278922) (end 153.23052 104.19848) (width 0.25) (layer "B.Cu") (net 20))
 (segment (start 153.23052 104.19848) (end 153.039 104.39) (width 0.25) (layer "B.Cu") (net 20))
 (segment (start 153.121202 101.169604) (end 153.23052 101.278922) (width 0.25) (layer "B.Cu") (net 20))
 (segment (start 155.212519 101.892487) (end 155.212519 100.799513) (width 0.2) (layer "F.Cu") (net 19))
 (segment (start 152.418519 100.311481) (end 152.146 100.584) (width 0.2) (layer "F.Cu") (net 19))
 (segment (start 154.724487 100.311481) (end 152.418519 100.311481) (width 0.2) (layer "F.Cu") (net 19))
 (segment (start 155.212519 100.799513) (end 154.724487 100.311481) (width 0.2) (layer "F.Cu") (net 19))
 (segment (start 154.994 102.111006) (end 155.212519 101.892487) (width 0.2) (layer "F.Cu") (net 19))
 (segment (start 154.994 102.513) (end 154.994 102.111006) (width 0.2) (layer "F.Cu") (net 19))
 (via (at 152.146 100.584) (size 0.8) (drill 0.4) (layers "F.Cu" "B.Cu") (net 19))
 (segment (start 152.781 103.728022) (end 152.619022 103.89) (width 0.25) (layer "B.Cu") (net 19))
 (segment (start 152.146 101.219) (end 152.781 101.854) (width 0.25) (layer "B.Cu") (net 19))
 (segment (start 152.146 100.584) (end 152.146 101.219) (width 0.25) (layer "B.Cu") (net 19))
 (segment (start 152.619022 103.89) (end 151.82 103.89) (width 0.25) (layer "B.Cu") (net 19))
 (segment (start 152.781 101.854) (end 152.781 103.728022) (width 0.25) (layer "B.Cu") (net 19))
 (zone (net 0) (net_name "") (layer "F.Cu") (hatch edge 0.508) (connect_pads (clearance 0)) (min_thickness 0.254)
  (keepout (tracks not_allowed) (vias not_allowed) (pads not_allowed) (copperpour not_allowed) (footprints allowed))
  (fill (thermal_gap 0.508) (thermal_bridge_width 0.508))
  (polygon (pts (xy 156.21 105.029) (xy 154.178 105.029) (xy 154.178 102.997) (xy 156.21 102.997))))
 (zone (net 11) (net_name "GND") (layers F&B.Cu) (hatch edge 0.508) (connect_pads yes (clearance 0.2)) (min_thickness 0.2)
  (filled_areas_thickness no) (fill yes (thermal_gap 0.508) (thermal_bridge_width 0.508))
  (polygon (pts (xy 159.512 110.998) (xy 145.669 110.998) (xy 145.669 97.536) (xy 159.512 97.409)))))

